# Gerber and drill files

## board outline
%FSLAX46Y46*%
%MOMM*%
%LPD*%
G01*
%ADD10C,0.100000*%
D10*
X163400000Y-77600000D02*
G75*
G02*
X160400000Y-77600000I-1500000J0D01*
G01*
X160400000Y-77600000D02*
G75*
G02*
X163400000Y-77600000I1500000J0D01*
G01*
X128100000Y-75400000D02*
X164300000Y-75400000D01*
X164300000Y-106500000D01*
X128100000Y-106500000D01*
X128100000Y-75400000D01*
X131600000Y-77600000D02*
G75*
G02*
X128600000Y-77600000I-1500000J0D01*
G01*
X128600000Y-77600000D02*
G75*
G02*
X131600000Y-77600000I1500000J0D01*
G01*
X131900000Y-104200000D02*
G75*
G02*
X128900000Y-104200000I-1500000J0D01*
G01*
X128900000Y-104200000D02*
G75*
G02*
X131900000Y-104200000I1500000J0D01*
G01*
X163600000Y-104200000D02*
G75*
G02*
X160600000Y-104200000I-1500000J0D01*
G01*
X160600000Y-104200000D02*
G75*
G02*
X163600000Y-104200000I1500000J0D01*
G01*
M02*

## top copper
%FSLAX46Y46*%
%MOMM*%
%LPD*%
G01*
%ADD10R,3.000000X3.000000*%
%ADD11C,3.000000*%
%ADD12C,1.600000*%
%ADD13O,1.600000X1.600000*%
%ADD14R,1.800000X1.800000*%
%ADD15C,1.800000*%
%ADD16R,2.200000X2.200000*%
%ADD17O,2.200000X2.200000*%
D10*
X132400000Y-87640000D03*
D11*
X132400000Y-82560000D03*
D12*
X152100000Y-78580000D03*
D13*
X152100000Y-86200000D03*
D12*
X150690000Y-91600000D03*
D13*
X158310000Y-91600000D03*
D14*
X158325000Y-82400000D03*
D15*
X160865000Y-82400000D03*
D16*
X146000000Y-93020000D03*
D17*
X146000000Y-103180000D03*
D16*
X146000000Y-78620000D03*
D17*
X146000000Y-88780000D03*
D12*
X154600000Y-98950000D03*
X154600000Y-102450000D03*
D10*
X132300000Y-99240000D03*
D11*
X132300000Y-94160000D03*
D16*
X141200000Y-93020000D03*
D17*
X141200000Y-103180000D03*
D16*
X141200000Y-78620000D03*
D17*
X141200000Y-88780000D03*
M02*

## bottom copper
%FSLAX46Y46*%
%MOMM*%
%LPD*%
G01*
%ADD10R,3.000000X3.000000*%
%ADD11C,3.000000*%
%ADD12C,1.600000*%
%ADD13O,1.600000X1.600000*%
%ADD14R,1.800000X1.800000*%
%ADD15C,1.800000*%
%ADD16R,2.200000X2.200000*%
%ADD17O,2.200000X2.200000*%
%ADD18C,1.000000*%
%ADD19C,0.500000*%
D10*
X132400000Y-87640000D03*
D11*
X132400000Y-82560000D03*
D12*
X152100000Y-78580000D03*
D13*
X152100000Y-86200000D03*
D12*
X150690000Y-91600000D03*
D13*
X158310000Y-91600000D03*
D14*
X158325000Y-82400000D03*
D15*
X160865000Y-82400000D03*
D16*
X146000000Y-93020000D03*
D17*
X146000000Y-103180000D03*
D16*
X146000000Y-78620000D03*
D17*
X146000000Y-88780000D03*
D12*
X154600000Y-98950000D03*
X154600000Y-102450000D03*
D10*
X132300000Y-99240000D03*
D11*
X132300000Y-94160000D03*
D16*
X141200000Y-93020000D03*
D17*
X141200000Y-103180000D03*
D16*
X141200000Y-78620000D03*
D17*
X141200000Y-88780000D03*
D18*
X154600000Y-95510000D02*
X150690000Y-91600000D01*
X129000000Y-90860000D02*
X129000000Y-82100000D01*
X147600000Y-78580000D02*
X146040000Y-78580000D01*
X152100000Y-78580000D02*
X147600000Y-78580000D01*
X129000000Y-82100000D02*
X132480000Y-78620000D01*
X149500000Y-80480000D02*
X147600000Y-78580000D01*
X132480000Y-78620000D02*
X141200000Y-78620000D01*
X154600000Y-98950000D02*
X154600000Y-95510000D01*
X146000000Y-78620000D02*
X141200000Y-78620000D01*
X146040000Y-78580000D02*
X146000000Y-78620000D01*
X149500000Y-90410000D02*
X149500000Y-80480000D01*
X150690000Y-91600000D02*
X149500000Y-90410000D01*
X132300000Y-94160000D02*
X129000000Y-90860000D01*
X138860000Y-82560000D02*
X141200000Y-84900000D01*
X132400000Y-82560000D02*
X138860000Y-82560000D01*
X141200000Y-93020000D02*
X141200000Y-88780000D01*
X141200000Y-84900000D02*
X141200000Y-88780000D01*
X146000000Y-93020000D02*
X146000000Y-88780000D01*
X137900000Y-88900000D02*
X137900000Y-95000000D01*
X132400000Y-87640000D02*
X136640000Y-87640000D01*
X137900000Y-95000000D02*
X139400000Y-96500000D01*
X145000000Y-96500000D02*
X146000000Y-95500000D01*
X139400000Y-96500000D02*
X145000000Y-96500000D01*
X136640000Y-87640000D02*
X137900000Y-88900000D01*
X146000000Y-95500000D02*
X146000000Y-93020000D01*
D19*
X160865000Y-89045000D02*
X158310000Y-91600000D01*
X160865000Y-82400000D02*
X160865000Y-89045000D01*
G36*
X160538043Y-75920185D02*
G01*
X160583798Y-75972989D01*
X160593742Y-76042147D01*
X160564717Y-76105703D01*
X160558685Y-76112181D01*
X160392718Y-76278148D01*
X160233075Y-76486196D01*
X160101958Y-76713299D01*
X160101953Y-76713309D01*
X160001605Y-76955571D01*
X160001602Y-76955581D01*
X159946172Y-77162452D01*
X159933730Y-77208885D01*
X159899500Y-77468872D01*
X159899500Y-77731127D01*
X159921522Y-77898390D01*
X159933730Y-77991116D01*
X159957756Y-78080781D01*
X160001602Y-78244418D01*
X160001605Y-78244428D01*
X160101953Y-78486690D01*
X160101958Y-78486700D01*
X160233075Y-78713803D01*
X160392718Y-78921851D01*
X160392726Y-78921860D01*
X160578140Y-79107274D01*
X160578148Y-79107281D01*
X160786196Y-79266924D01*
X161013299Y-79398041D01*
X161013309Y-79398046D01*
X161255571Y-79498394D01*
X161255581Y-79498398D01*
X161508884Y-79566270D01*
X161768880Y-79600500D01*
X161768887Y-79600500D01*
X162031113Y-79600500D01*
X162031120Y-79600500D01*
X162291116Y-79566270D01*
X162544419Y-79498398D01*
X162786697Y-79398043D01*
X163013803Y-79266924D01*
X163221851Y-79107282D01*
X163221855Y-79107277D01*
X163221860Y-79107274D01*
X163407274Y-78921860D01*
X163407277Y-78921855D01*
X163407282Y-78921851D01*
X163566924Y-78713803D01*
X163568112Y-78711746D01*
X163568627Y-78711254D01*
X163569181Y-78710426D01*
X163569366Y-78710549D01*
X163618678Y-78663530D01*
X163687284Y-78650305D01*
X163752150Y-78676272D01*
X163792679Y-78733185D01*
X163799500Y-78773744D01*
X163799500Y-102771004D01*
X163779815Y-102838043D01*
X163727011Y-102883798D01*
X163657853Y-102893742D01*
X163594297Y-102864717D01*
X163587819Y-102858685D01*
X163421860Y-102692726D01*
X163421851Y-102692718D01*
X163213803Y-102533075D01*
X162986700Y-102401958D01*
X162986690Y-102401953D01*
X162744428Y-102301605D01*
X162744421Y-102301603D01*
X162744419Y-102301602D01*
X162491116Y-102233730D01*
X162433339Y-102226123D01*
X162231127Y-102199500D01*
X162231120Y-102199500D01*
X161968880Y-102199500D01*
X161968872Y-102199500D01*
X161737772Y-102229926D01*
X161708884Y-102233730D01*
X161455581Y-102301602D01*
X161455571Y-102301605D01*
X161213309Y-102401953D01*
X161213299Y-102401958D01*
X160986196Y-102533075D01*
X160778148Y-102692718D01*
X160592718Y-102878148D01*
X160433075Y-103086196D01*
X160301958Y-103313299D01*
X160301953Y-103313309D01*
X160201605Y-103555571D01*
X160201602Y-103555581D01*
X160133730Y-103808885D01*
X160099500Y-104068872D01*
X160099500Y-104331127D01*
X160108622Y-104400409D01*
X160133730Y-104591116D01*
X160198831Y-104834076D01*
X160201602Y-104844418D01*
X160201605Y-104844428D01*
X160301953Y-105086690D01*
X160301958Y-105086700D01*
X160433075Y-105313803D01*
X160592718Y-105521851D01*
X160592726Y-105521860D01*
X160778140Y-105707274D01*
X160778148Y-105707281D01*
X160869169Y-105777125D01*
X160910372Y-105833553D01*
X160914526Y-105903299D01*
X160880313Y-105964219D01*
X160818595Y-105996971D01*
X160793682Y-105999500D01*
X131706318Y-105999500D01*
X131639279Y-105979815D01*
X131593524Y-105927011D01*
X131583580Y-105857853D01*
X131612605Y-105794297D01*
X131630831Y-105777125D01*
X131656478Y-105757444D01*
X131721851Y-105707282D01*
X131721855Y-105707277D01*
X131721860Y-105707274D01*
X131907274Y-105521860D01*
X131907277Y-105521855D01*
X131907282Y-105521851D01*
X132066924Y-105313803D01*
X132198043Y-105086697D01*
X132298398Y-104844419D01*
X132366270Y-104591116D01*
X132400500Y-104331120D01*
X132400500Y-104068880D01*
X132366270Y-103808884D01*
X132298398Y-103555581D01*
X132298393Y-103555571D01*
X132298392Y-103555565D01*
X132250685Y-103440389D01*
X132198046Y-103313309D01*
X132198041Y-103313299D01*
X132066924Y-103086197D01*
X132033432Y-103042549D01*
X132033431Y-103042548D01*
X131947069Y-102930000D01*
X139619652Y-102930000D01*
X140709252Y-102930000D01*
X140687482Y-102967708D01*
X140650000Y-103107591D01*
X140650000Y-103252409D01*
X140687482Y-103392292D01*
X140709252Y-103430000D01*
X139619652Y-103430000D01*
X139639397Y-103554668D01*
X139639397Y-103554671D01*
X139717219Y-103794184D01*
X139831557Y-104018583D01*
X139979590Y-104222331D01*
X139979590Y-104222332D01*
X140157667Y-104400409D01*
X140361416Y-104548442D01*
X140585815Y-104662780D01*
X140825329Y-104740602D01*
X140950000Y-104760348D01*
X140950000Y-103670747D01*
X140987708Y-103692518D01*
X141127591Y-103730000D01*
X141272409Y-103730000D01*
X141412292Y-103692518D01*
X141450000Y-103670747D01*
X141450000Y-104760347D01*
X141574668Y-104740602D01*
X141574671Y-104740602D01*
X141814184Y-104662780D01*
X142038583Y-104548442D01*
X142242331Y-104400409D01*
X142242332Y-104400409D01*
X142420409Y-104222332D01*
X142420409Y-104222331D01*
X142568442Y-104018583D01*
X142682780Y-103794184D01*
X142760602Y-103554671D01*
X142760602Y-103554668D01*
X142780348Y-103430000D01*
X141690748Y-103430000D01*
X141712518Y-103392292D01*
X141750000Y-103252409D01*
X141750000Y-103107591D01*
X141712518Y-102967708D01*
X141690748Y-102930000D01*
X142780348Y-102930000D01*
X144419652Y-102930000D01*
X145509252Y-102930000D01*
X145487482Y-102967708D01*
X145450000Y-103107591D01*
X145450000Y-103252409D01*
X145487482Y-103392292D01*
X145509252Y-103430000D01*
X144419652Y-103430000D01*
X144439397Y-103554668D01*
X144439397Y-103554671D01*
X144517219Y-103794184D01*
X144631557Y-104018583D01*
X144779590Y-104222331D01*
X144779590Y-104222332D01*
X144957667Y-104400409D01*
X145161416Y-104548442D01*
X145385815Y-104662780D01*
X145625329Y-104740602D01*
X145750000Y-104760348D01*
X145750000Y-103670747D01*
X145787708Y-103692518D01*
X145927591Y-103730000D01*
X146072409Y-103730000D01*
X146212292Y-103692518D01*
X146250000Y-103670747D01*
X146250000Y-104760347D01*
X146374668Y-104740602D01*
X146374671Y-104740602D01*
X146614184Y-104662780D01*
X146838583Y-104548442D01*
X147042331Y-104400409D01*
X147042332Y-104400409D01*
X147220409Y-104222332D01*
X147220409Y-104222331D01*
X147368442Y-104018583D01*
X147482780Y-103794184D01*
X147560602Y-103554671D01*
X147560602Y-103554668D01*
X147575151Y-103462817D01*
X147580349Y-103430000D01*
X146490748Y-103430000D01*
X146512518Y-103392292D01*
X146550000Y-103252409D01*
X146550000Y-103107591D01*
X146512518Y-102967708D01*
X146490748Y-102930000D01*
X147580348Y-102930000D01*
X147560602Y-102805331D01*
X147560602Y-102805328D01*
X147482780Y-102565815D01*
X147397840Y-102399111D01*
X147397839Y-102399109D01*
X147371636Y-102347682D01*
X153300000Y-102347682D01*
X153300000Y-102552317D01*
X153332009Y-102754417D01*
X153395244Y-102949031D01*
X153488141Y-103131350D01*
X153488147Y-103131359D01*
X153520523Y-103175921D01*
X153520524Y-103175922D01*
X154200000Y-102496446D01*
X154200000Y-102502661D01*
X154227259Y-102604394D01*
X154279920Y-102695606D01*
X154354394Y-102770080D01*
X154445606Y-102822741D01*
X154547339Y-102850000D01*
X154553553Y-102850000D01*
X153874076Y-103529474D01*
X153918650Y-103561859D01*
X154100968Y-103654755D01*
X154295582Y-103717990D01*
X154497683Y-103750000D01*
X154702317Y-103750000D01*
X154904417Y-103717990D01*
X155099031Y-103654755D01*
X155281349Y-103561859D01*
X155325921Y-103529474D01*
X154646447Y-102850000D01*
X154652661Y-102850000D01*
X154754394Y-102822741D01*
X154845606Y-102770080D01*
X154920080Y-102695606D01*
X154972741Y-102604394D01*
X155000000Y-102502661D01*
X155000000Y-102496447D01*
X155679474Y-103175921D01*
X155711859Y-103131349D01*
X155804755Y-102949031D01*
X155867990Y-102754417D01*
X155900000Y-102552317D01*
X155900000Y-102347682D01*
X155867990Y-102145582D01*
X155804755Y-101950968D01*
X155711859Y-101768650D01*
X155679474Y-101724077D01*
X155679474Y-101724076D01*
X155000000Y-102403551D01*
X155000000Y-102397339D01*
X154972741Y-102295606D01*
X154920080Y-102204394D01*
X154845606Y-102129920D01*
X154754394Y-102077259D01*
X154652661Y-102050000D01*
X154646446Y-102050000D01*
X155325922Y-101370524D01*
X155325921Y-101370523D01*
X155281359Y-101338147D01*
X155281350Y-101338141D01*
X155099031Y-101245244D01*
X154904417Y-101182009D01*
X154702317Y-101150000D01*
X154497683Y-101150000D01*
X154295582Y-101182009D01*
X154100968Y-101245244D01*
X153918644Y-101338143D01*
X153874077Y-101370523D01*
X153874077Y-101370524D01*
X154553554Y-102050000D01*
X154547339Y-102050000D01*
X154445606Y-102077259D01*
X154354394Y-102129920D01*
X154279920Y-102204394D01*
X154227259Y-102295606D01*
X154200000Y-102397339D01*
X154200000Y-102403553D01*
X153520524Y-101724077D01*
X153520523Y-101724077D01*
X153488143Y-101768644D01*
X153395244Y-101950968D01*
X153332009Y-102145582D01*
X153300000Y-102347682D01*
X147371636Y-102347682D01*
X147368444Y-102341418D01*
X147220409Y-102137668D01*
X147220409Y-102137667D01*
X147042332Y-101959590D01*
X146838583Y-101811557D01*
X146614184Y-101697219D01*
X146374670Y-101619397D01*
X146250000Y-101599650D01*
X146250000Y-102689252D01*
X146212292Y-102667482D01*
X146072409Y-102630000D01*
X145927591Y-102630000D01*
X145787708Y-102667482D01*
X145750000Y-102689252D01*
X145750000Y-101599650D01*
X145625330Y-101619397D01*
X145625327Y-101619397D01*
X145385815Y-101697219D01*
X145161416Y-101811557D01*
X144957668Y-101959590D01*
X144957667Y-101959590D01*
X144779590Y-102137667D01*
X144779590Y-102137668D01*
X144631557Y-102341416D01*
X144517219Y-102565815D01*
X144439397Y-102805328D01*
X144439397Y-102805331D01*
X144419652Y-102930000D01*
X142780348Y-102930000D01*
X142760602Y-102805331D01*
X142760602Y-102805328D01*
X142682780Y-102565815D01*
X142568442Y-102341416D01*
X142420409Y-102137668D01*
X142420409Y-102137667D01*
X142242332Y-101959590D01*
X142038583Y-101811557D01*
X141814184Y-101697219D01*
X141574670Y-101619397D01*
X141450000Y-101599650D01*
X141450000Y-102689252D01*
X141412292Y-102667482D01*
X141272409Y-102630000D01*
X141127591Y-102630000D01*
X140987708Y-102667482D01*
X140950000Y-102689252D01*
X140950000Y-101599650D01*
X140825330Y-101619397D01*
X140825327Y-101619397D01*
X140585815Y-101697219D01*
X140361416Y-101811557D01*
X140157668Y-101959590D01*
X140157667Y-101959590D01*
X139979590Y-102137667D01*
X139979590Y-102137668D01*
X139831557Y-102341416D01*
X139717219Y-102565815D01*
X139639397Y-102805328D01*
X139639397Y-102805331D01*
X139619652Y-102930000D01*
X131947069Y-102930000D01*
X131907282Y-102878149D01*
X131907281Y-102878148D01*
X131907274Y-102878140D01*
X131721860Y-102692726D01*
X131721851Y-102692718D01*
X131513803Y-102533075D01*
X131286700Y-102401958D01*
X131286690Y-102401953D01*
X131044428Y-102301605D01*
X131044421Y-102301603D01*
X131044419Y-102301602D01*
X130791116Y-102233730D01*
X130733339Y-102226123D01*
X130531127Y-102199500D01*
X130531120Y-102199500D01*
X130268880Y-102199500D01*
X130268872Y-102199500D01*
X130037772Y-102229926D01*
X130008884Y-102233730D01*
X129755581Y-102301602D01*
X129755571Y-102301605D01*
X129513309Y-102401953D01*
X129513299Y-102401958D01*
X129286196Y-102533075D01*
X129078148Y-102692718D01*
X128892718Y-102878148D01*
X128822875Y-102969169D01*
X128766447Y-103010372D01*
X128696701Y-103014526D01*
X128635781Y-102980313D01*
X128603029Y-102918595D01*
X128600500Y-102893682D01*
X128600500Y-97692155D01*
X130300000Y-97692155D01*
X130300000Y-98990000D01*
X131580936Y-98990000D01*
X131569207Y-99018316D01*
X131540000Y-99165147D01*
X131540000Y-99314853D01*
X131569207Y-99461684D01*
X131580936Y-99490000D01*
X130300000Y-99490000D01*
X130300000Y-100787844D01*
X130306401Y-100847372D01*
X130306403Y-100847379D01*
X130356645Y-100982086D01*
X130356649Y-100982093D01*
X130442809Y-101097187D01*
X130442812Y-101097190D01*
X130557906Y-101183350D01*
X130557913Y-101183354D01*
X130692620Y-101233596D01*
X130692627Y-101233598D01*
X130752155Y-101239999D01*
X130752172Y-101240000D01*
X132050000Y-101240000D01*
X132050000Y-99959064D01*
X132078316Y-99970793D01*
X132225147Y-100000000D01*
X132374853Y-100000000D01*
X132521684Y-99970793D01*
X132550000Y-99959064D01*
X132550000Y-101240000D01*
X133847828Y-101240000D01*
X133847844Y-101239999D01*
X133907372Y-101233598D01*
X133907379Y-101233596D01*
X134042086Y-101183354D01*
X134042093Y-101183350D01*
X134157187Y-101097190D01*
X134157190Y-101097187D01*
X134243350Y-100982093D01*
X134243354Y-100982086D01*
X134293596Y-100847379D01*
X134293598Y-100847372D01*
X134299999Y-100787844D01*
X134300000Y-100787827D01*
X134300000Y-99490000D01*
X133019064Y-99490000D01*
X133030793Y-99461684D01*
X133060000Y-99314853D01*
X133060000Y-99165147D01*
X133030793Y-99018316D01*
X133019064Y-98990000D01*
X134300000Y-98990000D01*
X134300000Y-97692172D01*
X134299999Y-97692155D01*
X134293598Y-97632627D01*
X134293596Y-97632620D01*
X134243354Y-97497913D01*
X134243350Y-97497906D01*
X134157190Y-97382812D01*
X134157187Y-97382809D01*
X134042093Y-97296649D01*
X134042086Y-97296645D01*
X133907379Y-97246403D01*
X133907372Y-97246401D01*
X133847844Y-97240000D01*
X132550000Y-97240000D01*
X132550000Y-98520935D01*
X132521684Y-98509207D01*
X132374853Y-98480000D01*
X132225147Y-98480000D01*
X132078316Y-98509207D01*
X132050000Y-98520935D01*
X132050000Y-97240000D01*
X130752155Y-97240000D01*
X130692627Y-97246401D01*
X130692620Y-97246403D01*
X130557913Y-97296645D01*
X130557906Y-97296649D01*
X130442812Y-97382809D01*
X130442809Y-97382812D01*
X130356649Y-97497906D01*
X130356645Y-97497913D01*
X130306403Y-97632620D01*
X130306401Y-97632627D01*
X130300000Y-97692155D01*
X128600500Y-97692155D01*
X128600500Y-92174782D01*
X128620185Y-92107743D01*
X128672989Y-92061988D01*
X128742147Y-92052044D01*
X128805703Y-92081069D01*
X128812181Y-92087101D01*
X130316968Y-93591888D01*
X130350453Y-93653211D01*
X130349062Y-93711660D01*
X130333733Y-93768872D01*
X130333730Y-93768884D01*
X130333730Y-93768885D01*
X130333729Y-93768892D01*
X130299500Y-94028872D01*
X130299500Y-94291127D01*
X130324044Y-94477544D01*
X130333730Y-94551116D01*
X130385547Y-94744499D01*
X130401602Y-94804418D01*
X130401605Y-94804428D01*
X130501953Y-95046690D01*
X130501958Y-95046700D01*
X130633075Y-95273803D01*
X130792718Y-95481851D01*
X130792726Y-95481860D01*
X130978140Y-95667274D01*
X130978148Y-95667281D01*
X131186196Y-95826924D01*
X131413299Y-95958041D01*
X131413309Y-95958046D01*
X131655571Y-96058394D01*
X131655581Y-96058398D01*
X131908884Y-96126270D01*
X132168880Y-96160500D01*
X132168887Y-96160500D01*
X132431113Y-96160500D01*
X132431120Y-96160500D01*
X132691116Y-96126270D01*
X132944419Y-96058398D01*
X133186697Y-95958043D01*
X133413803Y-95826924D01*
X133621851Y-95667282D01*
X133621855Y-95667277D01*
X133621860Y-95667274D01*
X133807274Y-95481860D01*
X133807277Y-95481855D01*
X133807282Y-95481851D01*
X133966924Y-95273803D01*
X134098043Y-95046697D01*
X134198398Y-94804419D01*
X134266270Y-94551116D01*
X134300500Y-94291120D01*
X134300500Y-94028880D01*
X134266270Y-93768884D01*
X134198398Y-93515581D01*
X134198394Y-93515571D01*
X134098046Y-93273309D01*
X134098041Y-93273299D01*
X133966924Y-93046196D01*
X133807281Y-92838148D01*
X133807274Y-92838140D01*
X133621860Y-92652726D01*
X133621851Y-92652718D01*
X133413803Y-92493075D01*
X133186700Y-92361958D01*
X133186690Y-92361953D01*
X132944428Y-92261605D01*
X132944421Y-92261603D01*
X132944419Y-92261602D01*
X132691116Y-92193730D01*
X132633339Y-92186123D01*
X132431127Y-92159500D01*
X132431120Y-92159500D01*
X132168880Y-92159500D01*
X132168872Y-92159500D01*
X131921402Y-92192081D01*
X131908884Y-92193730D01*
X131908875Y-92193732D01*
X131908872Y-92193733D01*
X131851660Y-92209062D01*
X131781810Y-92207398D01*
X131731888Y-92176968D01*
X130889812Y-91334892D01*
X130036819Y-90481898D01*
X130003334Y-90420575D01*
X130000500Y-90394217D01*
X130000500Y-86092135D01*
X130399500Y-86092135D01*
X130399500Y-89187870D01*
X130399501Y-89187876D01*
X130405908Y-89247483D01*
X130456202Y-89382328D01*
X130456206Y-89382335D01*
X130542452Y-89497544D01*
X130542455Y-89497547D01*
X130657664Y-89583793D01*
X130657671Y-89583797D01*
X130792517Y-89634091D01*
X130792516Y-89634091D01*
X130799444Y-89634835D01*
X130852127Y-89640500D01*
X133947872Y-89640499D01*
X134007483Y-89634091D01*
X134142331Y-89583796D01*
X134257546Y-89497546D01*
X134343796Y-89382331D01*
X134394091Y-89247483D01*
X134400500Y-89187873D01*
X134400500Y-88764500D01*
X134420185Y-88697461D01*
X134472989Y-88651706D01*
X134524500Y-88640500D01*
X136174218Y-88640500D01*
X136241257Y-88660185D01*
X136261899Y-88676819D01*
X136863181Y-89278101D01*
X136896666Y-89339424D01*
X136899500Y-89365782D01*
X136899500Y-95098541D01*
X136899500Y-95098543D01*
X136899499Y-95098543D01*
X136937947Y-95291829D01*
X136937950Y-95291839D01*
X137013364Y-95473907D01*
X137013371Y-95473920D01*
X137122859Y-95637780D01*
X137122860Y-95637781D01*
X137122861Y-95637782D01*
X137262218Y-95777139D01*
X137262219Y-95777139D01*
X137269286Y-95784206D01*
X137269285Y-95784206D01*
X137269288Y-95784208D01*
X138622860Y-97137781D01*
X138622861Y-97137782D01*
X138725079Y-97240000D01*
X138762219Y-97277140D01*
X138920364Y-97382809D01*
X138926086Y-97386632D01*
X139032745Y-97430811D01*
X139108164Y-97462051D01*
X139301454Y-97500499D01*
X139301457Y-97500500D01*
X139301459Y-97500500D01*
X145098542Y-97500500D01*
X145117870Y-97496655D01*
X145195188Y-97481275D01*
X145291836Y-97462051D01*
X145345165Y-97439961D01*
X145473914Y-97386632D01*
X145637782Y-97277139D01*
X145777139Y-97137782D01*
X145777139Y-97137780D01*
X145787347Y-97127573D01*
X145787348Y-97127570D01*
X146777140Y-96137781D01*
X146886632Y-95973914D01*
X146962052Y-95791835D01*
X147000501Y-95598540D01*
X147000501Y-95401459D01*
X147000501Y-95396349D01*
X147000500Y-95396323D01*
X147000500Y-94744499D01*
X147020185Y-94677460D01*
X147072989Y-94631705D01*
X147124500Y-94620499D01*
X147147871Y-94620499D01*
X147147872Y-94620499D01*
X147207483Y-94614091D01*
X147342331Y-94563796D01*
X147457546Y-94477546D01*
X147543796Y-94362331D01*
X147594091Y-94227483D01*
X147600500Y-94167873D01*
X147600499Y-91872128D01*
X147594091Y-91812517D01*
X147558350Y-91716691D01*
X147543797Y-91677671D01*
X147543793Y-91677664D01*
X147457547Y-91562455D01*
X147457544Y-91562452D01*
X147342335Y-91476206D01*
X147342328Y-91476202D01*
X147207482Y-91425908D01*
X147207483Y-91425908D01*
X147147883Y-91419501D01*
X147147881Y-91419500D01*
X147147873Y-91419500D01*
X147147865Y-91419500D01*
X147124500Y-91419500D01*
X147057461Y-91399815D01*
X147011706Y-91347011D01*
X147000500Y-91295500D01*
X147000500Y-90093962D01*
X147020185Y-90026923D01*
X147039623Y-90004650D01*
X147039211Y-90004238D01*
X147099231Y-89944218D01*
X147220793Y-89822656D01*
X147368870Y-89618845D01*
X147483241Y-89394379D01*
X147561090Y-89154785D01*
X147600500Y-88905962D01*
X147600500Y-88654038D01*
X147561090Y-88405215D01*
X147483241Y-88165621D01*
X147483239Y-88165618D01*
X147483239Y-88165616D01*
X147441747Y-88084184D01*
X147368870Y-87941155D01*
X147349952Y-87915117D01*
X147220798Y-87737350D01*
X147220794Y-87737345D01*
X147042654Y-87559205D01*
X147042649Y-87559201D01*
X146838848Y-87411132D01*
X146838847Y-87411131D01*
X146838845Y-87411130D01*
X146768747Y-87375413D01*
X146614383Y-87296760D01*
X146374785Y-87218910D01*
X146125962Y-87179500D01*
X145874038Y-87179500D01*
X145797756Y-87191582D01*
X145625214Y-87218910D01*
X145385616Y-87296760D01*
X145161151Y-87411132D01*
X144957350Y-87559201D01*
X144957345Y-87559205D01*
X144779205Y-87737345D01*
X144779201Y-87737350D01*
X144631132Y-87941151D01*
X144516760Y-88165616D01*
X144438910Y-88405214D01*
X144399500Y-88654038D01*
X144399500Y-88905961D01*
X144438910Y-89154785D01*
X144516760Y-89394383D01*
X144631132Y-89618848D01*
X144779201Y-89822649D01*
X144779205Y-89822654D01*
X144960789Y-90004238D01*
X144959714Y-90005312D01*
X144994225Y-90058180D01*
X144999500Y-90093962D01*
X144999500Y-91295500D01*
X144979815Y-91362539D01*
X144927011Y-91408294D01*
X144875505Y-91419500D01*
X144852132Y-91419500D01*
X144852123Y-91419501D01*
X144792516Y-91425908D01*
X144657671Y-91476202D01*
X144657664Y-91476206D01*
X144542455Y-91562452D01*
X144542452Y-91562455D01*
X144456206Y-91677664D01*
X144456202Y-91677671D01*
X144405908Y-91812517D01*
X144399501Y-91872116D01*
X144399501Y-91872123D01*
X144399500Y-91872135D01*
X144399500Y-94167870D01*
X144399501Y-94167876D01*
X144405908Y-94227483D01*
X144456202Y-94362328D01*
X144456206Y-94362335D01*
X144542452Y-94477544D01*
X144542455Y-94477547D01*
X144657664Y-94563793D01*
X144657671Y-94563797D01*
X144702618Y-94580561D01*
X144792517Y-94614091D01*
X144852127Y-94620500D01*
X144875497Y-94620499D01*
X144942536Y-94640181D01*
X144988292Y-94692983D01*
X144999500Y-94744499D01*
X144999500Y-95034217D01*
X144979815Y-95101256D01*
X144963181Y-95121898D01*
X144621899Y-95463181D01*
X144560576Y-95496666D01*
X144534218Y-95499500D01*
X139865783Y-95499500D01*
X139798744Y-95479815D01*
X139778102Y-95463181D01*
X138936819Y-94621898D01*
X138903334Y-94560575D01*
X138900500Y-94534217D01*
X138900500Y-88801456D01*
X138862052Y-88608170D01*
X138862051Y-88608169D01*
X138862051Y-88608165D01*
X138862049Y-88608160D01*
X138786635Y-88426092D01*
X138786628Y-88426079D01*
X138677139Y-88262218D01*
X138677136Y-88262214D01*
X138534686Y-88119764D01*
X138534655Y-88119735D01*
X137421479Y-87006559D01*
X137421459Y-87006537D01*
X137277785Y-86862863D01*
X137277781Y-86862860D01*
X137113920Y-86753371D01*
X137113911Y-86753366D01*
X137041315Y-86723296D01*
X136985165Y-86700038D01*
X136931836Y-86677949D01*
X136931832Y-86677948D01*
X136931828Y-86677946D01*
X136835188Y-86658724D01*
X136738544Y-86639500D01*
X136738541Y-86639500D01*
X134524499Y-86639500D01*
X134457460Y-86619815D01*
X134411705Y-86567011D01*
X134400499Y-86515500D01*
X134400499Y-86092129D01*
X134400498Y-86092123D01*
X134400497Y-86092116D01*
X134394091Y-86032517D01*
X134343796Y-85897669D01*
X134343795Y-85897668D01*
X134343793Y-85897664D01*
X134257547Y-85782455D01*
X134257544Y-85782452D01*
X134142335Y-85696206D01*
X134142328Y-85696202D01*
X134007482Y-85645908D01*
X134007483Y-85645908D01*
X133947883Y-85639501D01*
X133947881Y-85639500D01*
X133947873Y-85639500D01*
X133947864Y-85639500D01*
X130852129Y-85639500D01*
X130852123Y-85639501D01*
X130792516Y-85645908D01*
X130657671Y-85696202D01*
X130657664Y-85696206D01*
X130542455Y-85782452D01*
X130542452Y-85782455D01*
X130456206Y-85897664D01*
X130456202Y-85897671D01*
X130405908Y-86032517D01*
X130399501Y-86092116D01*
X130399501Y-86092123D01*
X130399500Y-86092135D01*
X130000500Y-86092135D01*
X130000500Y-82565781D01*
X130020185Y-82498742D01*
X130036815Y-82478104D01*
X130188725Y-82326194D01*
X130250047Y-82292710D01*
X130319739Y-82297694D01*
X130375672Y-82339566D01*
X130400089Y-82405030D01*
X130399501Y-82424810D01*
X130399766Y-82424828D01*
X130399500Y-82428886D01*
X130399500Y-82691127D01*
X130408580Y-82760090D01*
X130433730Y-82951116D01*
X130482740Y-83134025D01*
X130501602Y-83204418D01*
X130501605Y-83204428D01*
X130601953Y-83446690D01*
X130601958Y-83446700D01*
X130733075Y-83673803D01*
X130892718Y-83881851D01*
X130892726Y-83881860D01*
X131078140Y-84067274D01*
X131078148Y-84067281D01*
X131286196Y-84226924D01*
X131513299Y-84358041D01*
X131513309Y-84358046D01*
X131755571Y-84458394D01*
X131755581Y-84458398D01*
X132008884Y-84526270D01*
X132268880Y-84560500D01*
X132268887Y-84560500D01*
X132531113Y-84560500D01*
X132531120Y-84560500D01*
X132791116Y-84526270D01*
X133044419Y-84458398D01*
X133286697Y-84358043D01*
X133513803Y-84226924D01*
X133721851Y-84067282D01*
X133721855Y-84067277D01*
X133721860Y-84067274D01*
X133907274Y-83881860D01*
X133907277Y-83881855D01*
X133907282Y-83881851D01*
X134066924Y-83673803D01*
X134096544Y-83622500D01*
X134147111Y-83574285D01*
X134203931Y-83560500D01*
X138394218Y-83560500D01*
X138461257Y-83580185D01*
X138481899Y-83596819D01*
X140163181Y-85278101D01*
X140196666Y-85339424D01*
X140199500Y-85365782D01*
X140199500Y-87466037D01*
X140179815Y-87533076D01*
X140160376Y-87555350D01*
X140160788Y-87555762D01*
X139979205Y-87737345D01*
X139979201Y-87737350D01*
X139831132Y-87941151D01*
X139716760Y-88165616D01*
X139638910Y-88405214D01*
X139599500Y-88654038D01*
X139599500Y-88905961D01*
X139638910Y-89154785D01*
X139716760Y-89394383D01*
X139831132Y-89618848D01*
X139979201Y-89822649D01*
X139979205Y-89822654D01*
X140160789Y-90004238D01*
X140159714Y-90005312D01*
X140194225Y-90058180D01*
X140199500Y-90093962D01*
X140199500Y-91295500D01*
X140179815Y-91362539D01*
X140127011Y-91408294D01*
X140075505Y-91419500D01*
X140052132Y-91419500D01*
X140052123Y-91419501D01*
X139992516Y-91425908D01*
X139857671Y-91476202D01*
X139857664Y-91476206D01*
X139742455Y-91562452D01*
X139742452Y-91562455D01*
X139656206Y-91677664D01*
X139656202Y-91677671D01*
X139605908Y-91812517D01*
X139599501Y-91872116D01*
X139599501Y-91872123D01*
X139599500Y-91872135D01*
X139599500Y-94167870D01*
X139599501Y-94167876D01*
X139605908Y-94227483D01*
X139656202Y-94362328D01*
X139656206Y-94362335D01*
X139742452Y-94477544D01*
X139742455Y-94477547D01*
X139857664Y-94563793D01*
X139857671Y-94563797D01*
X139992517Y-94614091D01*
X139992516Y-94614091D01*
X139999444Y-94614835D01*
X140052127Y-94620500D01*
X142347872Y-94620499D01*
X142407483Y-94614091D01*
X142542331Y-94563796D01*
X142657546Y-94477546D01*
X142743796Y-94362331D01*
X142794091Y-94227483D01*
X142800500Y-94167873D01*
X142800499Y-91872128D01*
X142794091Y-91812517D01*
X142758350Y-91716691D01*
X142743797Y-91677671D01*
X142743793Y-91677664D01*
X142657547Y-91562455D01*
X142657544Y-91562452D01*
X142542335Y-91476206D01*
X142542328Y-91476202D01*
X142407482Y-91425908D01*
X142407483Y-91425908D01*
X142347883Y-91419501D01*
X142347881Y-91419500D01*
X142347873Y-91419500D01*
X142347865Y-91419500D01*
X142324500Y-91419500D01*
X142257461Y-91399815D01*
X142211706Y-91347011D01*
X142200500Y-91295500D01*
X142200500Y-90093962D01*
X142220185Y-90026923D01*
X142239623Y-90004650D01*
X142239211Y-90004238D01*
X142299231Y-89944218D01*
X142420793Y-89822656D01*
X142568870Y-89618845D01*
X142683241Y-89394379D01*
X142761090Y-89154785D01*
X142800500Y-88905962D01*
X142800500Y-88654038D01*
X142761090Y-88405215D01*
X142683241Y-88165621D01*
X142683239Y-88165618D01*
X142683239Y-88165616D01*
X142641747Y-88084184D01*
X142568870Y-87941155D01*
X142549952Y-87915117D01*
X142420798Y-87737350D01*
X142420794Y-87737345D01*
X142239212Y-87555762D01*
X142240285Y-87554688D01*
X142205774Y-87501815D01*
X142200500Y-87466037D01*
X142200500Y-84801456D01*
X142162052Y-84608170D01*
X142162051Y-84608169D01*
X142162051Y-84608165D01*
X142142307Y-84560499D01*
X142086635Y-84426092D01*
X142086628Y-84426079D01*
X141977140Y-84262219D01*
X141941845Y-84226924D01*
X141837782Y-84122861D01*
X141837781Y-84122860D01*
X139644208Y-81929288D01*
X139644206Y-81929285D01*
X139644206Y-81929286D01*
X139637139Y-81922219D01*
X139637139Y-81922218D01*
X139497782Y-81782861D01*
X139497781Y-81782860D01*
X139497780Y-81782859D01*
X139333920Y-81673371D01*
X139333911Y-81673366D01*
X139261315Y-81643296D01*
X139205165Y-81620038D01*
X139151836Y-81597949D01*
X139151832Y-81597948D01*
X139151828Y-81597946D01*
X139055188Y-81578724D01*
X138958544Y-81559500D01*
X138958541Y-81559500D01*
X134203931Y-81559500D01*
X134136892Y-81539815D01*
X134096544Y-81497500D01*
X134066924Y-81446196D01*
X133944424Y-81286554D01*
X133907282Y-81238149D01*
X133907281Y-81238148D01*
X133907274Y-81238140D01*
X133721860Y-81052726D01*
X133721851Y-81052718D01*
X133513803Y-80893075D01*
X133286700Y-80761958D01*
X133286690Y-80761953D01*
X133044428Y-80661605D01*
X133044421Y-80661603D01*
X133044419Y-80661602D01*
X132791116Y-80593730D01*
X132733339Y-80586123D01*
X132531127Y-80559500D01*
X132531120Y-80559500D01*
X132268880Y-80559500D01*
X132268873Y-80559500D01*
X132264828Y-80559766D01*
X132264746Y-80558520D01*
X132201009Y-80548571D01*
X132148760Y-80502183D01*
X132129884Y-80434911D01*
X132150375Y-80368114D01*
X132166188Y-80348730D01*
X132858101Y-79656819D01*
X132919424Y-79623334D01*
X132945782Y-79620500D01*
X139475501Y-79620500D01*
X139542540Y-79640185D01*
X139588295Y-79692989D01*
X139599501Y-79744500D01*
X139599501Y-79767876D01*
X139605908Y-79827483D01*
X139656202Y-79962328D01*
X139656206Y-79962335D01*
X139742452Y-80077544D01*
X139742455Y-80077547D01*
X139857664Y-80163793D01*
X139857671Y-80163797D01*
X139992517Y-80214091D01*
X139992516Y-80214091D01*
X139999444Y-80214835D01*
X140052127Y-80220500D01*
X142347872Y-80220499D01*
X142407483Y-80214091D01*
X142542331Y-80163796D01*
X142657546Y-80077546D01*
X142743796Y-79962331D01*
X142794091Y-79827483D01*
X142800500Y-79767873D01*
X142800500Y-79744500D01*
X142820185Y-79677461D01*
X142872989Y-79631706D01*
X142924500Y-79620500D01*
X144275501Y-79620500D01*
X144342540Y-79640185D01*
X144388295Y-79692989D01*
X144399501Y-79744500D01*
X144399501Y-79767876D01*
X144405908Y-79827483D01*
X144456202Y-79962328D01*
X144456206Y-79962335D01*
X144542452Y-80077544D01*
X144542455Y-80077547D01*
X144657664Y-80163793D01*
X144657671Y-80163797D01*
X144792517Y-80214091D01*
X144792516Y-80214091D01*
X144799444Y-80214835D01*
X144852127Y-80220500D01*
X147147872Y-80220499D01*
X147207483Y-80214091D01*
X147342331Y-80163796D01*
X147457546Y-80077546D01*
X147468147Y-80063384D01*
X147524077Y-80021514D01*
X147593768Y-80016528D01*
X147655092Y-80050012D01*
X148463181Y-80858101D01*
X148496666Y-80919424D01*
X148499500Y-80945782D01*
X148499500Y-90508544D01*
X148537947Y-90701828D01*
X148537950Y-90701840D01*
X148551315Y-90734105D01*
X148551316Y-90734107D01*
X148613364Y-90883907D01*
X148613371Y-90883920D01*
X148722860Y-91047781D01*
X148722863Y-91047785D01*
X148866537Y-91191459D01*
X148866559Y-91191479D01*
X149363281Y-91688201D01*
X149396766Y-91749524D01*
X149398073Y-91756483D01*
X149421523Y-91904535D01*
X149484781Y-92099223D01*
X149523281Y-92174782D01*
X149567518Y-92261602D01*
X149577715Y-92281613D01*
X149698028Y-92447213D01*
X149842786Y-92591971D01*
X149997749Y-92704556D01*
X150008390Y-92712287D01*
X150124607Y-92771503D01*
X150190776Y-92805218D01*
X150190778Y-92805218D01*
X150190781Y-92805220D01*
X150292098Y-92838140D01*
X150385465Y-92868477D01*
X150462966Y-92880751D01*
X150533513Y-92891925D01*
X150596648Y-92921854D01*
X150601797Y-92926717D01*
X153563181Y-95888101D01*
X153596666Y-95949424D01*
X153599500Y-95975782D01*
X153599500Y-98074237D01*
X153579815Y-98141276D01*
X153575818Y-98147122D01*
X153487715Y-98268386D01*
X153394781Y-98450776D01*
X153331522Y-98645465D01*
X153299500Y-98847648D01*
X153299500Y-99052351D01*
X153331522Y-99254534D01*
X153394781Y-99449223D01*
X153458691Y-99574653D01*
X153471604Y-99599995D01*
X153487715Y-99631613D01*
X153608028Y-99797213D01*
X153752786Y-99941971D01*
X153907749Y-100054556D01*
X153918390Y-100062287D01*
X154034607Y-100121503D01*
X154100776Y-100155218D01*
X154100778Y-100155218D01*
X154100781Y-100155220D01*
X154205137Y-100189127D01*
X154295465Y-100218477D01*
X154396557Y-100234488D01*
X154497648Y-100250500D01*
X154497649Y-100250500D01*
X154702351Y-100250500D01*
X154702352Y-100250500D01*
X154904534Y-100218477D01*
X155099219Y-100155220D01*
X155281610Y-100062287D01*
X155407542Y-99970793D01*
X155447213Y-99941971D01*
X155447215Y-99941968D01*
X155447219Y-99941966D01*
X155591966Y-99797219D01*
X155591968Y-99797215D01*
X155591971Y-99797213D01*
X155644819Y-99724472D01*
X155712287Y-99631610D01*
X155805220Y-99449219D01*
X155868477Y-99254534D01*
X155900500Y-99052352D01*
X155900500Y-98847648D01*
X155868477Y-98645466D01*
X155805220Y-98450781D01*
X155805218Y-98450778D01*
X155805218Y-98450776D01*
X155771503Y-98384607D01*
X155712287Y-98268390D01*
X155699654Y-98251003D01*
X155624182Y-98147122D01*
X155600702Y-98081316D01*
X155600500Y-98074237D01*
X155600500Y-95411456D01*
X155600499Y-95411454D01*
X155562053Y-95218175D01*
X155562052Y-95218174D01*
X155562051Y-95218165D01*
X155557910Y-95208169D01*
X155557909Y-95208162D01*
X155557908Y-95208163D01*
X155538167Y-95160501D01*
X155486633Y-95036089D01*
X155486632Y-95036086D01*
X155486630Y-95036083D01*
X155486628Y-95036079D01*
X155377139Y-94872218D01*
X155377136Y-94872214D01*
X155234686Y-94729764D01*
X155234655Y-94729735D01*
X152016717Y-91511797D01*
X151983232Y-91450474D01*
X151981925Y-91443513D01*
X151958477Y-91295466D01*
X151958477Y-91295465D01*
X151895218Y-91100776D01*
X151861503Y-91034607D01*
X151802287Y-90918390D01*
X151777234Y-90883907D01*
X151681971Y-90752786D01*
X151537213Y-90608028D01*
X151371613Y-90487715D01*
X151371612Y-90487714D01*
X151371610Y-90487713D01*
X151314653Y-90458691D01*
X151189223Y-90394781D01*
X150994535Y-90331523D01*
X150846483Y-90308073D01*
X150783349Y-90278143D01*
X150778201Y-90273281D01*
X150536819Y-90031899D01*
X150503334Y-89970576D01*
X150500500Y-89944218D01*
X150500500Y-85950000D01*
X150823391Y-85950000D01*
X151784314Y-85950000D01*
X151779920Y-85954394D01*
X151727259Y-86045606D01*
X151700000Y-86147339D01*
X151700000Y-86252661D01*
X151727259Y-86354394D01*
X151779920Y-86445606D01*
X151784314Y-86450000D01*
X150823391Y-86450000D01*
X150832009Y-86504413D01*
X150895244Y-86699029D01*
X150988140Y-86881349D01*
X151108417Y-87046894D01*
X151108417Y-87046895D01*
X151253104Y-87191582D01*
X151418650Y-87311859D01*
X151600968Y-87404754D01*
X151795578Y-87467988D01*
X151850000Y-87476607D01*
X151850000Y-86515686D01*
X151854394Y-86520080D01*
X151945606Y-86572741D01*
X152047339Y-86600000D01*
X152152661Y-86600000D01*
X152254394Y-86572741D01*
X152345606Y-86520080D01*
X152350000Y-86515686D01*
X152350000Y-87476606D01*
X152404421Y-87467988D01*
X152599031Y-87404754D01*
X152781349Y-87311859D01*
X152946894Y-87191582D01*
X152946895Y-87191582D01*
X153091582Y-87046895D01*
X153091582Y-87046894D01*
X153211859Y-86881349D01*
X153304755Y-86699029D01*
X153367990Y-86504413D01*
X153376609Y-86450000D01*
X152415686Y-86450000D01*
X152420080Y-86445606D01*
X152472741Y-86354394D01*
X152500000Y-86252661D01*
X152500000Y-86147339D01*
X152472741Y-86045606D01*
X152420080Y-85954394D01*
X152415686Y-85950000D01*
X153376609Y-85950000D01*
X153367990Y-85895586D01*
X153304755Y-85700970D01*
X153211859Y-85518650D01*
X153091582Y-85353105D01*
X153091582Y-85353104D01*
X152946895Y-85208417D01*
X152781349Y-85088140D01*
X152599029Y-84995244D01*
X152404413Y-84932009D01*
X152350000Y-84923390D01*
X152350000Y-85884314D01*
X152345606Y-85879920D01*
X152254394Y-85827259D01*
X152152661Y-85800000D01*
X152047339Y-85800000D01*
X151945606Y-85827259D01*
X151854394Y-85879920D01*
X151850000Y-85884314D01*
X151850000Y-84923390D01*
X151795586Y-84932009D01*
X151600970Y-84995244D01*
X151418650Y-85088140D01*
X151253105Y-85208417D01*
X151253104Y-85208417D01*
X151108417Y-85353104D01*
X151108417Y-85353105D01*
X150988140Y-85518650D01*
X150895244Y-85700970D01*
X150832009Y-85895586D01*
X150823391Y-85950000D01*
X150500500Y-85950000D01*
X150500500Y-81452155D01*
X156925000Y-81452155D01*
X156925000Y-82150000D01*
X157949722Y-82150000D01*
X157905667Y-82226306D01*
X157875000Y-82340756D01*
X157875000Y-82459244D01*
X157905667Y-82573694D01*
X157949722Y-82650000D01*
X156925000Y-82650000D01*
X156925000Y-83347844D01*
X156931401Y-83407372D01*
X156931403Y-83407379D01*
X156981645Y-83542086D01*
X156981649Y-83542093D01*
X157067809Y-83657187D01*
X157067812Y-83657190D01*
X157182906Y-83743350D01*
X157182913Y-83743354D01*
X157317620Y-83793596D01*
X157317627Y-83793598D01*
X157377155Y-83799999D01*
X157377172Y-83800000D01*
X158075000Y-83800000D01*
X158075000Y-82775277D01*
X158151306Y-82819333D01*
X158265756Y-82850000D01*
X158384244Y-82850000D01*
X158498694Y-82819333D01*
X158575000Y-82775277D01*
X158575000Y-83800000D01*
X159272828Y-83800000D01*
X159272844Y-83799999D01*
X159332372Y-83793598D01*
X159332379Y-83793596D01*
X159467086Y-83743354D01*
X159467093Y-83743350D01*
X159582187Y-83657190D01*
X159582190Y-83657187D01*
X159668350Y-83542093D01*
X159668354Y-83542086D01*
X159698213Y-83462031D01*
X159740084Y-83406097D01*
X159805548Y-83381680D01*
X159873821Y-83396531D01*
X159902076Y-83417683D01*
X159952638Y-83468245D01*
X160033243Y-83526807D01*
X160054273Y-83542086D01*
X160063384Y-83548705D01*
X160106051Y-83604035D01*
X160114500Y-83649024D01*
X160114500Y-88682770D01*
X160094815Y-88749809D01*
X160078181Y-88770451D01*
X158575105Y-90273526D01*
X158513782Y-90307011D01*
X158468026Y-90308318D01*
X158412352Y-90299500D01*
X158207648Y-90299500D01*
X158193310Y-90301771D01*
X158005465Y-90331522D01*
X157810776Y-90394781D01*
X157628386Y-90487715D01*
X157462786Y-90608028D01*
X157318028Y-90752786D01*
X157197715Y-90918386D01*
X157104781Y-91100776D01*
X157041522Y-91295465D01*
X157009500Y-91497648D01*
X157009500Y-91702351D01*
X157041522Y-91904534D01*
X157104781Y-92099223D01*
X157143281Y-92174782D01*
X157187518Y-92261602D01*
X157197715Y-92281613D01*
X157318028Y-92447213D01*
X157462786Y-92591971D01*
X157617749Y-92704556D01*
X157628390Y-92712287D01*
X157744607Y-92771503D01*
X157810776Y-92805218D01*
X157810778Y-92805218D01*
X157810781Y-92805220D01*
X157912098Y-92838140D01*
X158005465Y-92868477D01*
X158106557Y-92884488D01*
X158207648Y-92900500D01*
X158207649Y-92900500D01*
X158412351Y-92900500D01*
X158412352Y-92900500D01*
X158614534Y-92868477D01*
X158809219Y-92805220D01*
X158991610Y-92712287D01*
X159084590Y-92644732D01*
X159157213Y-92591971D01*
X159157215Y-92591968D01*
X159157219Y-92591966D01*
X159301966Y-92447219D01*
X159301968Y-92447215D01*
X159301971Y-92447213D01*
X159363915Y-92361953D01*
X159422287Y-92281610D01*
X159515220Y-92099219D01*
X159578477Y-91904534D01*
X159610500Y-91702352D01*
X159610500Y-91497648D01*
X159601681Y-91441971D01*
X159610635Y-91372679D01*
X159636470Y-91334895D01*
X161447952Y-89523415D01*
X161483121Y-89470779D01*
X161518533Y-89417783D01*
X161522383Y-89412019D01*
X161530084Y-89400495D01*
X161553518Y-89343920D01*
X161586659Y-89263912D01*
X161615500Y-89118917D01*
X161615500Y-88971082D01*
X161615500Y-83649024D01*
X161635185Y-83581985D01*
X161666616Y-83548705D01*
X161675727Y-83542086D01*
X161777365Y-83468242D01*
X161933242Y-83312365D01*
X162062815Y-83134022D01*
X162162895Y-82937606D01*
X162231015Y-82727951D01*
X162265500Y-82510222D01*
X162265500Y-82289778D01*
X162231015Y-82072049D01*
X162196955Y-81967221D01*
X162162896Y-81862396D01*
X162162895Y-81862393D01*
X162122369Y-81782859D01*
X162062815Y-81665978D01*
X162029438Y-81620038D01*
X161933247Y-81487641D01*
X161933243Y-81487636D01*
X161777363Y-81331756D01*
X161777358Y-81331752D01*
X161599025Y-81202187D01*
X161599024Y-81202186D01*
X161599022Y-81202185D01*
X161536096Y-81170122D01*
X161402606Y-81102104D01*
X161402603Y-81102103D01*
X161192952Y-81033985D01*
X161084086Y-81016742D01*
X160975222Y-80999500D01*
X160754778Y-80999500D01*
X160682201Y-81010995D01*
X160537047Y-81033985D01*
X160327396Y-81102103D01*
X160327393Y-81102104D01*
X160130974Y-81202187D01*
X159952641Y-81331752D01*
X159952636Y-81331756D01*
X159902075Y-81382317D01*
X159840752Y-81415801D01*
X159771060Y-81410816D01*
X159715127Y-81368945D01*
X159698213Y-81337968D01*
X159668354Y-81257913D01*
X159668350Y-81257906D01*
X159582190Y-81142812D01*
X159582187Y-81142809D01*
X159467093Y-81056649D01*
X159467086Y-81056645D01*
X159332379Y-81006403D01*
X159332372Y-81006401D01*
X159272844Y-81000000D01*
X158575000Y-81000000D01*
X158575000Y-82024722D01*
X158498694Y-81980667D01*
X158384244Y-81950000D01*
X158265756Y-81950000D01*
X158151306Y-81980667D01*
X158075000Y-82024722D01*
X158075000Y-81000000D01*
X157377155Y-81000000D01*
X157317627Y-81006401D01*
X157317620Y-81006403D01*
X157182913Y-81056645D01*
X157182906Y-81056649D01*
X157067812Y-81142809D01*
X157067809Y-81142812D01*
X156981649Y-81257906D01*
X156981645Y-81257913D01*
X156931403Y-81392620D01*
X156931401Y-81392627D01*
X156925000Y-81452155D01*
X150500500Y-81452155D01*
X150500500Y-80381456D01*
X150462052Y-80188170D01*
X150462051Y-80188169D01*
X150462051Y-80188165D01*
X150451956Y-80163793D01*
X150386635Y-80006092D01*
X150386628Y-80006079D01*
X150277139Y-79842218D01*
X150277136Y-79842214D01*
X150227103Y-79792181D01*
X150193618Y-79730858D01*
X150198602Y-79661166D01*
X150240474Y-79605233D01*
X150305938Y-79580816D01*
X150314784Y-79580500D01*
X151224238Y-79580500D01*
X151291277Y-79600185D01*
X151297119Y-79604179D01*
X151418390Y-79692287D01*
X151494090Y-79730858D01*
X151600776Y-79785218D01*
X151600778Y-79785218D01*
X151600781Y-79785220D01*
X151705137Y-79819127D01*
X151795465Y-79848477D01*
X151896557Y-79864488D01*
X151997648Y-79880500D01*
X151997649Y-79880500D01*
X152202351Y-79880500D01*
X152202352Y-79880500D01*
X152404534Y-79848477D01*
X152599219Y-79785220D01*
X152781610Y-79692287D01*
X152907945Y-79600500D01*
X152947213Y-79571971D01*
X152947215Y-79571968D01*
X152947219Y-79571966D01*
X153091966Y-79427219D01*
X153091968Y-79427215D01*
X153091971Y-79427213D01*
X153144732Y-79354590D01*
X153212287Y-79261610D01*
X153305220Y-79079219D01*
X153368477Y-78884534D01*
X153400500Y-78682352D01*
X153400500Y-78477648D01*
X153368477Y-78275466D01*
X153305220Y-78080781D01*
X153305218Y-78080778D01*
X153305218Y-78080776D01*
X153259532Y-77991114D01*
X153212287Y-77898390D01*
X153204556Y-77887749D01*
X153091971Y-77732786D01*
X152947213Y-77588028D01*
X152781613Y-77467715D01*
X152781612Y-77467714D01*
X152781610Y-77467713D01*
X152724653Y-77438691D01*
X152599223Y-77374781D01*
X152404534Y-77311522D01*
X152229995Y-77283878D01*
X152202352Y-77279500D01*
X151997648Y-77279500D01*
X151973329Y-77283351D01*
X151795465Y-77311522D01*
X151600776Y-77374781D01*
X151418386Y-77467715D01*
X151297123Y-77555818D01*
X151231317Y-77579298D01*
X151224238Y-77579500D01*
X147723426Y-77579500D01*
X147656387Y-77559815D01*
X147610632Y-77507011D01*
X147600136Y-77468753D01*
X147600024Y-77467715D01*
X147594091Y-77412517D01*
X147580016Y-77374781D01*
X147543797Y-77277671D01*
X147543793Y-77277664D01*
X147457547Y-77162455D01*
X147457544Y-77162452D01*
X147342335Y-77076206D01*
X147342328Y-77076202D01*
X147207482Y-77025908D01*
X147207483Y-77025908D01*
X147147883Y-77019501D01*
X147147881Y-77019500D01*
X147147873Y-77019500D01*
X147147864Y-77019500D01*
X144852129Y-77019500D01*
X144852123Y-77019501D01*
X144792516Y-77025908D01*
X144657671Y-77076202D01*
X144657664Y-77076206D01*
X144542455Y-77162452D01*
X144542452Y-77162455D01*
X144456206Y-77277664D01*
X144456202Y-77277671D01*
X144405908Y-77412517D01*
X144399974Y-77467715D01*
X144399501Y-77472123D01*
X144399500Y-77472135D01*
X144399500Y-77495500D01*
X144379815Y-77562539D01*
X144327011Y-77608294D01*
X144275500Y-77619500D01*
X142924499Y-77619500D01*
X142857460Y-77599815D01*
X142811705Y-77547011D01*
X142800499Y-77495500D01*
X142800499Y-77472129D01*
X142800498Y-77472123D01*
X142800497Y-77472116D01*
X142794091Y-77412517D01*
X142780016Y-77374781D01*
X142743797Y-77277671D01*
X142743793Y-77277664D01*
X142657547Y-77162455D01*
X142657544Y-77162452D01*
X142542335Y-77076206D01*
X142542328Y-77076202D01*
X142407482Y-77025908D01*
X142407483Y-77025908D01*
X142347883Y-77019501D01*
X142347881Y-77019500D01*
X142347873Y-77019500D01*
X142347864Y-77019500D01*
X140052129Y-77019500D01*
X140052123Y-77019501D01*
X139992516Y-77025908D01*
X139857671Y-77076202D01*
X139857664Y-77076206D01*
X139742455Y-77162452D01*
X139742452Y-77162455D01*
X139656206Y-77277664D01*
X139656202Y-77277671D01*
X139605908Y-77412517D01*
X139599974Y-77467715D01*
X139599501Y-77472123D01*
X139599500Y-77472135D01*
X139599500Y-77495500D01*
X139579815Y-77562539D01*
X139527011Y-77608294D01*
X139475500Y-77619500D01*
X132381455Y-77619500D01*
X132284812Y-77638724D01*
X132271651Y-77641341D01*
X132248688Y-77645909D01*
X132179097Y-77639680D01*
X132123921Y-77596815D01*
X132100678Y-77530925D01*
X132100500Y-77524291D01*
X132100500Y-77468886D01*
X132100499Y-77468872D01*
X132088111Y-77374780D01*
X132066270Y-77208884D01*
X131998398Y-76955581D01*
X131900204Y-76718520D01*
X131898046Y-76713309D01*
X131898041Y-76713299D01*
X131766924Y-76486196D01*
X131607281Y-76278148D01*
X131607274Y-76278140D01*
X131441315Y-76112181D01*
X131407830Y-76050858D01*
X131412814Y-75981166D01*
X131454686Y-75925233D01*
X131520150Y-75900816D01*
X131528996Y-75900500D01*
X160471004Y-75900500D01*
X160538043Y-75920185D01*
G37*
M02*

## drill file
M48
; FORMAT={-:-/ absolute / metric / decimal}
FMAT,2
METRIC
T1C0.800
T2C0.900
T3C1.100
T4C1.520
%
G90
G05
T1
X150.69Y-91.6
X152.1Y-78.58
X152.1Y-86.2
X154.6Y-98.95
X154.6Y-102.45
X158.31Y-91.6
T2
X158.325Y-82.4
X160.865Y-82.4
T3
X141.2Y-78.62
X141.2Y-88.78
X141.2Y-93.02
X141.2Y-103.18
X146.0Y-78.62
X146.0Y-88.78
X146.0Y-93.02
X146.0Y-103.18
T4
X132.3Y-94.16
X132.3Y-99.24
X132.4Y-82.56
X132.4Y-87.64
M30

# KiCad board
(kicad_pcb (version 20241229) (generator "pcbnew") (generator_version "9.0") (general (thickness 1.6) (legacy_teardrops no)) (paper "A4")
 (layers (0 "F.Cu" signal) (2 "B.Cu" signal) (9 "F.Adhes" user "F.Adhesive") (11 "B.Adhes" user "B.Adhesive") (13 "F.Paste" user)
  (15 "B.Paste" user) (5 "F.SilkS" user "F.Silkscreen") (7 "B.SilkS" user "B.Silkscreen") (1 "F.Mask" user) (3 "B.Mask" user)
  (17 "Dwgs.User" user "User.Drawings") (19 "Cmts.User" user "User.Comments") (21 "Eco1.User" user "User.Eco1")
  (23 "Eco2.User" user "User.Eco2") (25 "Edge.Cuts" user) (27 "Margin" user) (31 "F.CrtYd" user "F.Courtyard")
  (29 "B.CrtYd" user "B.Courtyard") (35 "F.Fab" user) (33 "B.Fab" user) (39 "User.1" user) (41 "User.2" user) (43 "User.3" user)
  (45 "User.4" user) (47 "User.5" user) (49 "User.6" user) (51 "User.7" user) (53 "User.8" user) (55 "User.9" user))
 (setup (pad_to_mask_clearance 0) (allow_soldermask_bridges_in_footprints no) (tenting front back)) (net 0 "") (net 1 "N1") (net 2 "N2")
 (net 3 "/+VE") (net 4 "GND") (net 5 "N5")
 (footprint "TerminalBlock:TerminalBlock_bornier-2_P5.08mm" (layer "F.Cu") (at 132.4 87.64 90)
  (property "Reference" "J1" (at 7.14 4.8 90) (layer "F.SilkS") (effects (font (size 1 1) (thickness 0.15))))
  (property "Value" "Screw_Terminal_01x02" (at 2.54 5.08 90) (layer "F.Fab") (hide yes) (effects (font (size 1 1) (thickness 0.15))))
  (pad "1" thru_hole rect (at 0 0 90) (size 3 3) (drill 1.52) (layers "*.Cu" "*.Mask") (remove_unused_layers no) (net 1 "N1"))
  (pad "2" thru_hole circle (at 5.08 0 90) (size 3 3) (drill 1.52) (layers "*.Cu" "*.Mask") (remove_unused_layers no) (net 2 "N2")))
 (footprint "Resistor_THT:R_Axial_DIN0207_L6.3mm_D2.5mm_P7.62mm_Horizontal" (layer "F.Cu") (at 152.1 78.58 -90)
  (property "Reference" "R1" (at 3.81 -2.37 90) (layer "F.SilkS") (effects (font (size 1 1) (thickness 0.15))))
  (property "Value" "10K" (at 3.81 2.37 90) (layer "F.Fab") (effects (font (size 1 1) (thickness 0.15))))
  (pad "1" thru_hole circle (at 0 0 270) (size 1.6 1.6) (drill 0.8) (layers "*.Cu" "*.Mask") (remove_unused_layers no) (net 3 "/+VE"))
  (pad "2" thru_hole oval (at 7.62 0 270) (size 1.6 1.6) (drill 0.8) (layers "*.Cu" "*.Mask") (remove_unused_layers no) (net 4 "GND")))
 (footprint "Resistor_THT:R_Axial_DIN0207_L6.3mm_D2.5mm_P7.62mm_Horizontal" (layer "F.Cu") (at 150.69 91.6)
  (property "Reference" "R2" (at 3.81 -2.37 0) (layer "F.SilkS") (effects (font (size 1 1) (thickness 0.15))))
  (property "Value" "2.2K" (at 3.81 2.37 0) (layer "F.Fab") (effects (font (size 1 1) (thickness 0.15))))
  (pad "1" thru_hole circle (at 0 0) (size 1.6 1.6) (drill 0.8) (layers "*.Cu" "*.Mask") (remove_unused_layers no) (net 3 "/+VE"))
  (pad "2" thru_hole oval (at 7.62 0) (size 1.6 1.6) (drill 0.8) (layers "*.Cu" "*.Mask") (remove_unused_layers no) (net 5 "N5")))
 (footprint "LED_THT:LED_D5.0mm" (layer "F.Cu") (at 158.325 82.4)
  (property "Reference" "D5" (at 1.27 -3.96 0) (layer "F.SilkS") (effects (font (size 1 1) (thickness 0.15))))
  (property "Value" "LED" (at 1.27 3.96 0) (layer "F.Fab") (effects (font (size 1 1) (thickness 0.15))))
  (pad "1" thru_hole rect (at 0 0) (size 1.8 1.8) (drill 0.9) (layers "*.Cu" "*.Mask") (remove_unused_layers no) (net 4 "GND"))
  (pad "2" thru_hole circle (at 2.54 0) (size 1.8 1.8) (drill 0.9) (layers "*.Cu" "*.Mask") (remove_unused_layers no) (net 5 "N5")))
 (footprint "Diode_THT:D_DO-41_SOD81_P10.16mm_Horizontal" (layer "F.Cu") (at 146 93.02 -90)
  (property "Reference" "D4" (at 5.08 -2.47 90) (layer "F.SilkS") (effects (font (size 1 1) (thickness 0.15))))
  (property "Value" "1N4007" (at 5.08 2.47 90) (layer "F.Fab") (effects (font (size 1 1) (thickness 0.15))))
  (pad "1" thru_hole rect (at 0 0 270) (size 2.2 2.2) (drill 1.1) (layers "*.Cu" "*.Mask") (remove_unused_layers no) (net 1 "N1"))
  (pad "2" thru_hole oval (at 10.16 0 270) (size 2.2 2.2) (drill 1.1) (layers "*.Cu" "*.Mask") (remove_unused_layers no) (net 4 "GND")))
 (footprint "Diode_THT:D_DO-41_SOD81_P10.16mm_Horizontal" (layer "F.Cu") (at 146 78.62 -90)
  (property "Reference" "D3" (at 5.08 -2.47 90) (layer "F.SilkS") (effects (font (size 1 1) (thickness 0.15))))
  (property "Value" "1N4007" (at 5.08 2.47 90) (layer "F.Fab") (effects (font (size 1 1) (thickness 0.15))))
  (pad "1" thru_hole rect (at 0 0 270) (size 2.2 2.2) (drill 1.1) (layers "*.Cu" "*.Mask") (remove_unused_layers no) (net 3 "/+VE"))
  (pad "2" thru_hole oval (at 10.16 0 270) (size 2.2 2.2) (drill 1.1) (layers "*.Cu" "*.Mask") (remove_unused_layers no) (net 1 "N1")))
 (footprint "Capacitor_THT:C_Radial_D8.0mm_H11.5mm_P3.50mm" (layer "F.Cu") (at 154.6 98.95 -90)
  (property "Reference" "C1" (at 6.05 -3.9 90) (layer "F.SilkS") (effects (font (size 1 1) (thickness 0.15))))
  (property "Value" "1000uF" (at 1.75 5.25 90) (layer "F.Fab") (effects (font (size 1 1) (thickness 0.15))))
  (pad "1" thru_hole circle (at 0 0 270) (size 1.6 1.6) (drill 0.8) (layers "*.Cu" "*.Mask") (remove_unused_layers no) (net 3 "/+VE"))
  (pad "2" thru_hole circle (at 3.5 0 270) (size 1.6 1.6) (drill 0.8) (layers "*.Cu" "*.Mask") (remove_unused_layers no) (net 4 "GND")))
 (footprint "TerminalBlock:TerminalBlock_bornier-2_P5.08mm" (layer "F.Cu") (at 132.3 99.24 90)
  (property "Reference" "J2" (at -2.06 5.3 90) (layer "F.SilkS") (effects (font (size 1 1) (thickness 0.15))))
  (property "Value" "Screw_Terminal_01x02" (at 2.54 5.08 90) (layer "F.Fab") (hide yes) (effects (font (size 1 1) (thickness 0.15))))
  (pad "1" thru_hole rect (at 0 0 90) (size 3 3) (drill 1.52) (layers "*.Cu" "*.Mask") (remove_unused_layers no) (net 4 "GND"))
  (pad "2" thru_hole circle (at 5.08 0 90) (size 3 3) (drill 1.52) (layers "*.Cu" "*.Mask") (remove_unused_layers no) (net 3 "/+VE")))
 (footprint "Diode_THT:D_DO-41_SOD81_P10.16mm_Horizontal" (layer "F.Cu") (at 141.2 93.02 -90)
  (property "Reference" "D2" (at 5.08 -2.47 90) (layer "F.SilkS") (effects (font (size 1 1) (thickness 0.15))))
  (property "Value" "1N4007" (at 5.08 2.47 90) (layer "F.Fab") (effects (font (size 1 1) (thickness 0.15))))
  (pad "1" thru_hole rect (at 0 0 270) (size 2.2 2.2) (drill 1.1) (layers "*.Cu" "*.Mask") (remove_unused_layers no) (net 2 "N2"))
  (pad "2" thru_hole oval (at 10.16 0 270) (size 2.2 2.2) (drill 1.1) (layers "*.Cu" "*.Mask") (remove_unused_layers no) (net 4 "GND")))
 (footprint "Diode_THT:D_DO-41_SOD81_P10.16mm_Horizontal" (layer "F.Cu") (at 141.2 78.62 -90)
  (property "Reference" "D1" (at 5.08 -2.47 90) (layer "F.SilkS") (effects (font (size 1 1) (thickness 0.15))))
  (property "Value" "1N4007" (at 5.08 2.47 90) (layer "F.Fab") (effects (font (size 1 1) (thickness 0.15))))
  (pad "1" thru_hole rect (at 0 0 270) (size 2.2 2.2) (drill 1.1) (layers "*.Cu" "*.Mask") (remove_unused_layers no) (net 3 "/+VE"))
  (pad "2" thru_hole oval (at 10.16 0 270) (size 2.2 2.2) (drill 1.1) (layers "*.Cu" "*.Mask") (remove_unused_layers no) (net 2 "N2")))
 (gr_circle (center 161.9 77.6) (end 163.4 77.6) (stroke (width 0.1) (type default)) (fill no) (layer "Edge.Cuts"))
 (gr_rect (start 128.1 75.4) (end 164.3 106.5) (stroke (width 0.1) (type default)) (fill no) (layer "Edge.Cuts"))
 (gr_circle (center 130.1 77.6) (end 131.6 77.6) (stroke (width 0.1) (type default)) (fill no) (layer "Edge.Cuts"))
 (gr_circle (center 130.4 104.2) (end 131.9 104.2) (stroke (width 0.1) (type default)) (fill no) (layer "Edge.Cuts"))
 (gr_circle (center 162.1 104.2) (end 163.6 104.2) (stroke (width 0.1) (type default)) (fill no) (layer "Edge.Cuts"))
 (segment (start 154.6 95.51) (end 150.69 91.6) (width 1) (layer "B.Cu") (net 3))
 (segment (start 129 90.86) (end 129 82.1) (width 1) (layer "B.Cu") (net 3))
 (segment (start 147.6 78.58) (end 146.04 78.58) (width 1) (layer "B.Cu") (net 3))
 (segment (start 152.1 78.58) (end 147.6 78.58) (width 1) (layer "B.Cu") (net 3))
 (segment (start 129 82.1) (end 132.48 78.62) (width 1) (layer "B.Cu") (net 3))
 (segment (start 149.5 80.48) (end 147.6 78.58) (width 1) (layer "B.Cu") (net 3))
 (segment (start 132.48 78.62) (end 141.2 78.62) (width 1) (layer "B.Cu") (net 3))
 (segment (start 154.6 98.95) (end 154.6 95.51) (width 1) (layer "B.Cu") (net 3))
 (segment (start 146 78.62) (end 141.2 78.62) (width 1) (layer "B.Cu") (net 3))
 (segment (start 146.04 78.58) (end 146 78.62) (width 1) (layer "B.Cu") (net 3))
 (segment (start 149.5 90.41) (end 149.5 80.48) (width 1) (layer "B.Cu") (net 3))
 (segment (start 150.69 91.6) (end 149.5 90.41) (width 1) (layer "B.Cu") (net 3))
 (segment (start 132.3 94.16) (end 129 90.86) (width 1) (layer "B.Cu") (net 3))
 (segment (start 138.86 82.56) (end 141.2 84.9) (width 1) (layer "B.Cu") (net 2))
 (segment (start 132.4 82.56) (end 138.86 82.56) (width 1) (layer "B.Cu") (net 2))
 (segment (start 141.2 93.02) (end 141.2 88.78) (width 1) (layer "B.Cu") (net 2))
 (segment (start 141.2 84.9) (end 141.2 88.78) (width 1) (layer "B.Cu") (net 2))
 (segment (start 146 93.02) (end 146 88.78) (width 1) (layer "B.Cu") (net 1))
 (segment (start 137.9 88.9) (end 137.9 95) (width 1) (layer "B.Cu") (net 1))
 (segment (start 132.4 87.64) (end 136.64 87.64) (width 1) (layer "B.Cu") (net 1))
 (segment (start 137.9 95) (end 139.4 96.5) (width 1) (layer "B.Cu") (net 1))
 (segment (start 145 96.5) (end 146 95.5) (width 1) (layer "B.Cu") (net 1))
 (segment (start 139.4 96.5) (end 145 96.5) (width 1) (layer "B.Cu") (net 1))
 (segment (start 136.64 87.64) (end 137.9 88.9) (width 1) (layer "B.Cu") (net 1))
 (segment (start 146 95.5) (end 146 93.02) (width 1) (layer "B.Cu") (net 1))
 (segment (start 160.865 89.045) (end 158.31 91.6) (width 0.5) (layer "B.Cu") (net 5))
 (segment (start 160.865 82.4) (end 160.865 89.045) (width 0.5) (layer "B.Cu") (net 5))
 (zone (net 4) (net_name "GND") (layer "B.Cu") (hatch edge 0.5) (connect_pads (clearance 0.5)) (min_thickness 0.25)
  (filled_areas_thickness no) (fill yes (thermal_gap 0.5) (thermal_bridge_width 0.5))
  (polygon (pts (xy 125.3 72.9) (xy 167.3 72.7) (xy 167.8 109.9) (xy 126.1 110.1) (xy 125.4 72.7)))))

